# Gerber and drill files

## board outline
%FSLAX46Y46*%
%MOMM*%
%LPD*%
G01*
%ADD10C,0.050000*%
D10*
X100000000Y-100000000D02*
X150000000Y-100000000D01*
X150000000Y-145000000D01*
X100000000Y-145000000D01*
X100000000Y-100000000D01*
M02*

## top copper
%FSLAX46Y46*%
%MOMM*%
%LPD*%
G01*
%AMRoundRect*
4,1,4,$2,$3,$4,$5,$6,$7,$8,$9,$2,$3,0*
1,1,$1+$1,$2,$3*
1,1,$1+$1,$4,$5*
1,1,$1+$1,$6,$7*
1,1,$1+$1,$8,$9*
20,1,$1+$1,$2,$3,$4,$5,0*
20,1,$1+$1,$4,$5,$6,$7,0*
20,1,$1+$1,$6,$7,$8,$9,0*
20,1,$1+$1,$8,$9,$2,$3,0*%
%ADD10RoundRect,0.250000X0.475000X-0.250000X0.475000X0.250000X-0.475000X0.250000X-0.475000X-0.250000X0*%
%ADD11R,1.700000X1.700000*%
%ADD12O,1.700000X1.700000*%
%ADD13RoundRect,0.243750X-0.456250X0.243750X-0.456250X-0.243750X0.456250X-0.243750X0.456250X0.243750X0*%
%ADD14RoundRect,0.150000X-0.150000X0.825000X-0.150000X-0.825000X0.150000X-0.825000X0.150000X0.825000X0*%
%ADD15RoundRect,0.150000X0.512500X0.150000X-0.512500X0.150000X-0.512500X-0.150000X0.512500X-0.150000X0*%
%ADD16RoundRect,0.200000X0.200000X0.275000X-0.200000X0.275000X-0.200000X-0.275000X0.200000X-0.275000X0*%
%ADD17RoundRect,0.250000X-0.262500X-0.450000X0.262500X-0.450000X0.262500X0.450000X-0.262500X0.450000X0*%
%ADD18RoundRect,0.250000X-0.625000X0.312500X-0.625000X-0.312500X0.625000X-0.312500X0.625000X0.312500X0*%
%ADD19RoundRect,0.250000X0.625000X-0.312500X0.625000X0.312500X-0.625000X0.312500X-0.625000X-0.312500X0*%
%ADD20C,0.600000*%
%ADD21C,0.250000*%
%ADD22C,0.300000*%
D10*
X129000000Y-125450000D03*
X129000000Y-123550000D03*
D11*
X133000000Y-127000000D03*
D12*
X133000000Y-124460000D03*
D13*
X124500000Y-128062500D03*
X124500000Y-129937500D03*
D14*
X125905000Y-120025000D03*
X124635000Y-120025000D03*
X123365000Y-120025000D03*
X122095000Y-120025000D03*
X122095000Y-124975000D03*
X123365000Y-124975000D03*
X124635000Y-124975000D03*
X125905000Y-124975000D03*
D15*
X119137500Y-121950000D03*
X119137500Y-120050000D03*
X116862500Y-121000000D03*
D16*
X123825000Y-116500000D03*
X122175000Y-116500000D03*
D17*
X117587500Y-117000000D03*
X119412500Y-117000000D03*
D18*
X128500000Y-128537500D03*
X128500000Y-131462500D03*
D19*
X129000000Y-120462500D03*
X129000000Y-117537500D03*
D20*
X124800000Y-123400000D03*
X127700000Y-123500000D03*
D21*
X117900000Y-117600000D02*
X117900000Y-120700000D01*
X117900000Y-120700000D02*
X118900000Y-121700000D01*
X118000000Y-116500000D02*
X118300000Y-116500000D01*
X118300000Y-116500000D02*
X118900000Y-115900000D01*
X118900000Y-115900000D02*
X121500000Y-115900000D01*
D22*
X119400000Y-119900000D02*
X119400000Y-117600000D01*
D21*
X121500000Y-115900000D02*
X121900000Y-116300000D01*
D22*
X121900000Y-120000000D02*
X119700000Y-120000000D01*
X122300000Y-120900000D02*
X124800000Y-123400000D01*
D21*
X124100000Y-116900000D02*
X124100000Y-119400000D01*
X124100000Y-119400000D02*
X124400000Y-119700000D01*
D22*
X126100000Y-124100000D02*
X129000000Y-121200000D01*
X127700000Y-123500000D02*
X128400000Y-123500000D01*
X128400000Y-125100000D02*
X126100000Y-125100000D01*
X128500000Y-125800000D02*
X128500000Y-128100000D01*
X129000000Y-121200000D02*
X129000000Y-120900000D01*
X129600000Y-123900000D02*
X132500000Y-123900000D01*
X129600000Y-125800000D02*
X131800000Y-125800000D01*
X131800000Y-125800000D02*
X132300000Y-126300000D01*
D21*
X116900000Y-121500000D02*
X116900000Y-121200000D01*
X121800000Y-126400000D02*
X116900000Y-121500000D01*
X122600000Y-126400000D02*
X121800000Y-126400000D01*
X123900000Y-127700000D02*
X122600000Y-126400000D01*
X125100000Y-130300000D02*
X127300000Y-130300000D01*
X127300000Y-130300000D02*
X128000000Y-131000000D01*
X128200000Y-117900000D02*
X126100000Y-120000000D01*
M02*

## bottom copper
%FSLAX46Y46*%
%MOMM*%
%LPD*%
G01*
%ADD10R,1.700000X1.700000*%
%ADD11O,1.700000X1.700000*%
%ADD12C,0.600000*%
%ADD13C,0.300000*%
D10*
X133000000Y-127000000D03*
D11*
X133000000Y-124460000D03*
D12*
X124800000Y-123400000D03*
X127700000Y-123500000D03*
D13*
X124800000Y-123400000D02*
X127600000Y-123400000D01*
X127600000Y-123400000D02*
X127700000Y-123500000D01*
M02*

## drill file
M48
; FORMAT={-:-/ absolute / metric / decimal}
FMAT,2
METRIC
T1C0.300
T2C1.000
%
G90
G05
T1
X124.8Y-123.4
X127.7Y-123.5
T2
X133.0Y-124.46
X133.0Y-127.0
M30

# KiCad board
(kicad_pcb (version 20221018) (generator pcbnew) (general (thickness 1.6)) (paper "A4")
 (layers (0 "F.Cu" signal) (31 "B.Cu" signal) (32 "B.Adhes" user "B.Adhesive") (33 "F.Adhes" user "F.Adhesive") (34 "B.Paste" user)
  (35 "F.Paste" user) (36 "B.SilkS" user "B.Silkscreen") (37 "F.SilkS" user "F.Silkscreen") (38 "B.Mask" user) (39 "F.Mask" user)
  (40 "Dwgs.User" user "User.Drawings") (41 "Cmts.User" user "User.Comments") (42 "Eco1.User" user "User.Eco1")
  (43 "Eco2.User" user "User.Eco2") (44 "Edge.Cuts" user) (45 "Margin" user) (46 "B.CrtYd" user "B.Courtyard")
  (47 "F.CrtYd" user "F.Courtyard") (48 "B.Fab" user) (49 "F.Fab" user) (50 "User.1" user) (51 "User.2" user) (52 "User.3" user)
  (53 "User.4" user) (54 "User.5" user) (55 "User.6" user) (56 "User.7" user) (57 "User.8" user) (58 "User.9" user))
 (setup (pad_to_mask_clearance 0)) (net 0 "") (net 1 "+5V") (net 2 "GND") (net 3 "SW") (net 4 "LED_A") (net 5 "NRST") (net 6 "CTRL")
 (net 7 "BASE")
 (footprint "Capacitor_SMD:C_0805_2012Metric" (layer "F.Cu") (at 129 124.5 90)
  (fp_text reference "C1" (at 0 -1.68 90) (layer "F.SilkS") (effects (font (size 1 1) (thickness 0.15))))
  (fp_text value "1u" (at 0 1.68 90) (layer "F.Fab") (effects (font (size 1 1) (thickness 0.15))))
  (pad "1" smd roundrect (at -0.95 0 90) (size 1 1.45) (layers "F.Cu" "F.Paste" "F.Mask") (roundrect_rratio 0.25) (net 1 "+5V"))
  (pad "2" smd roundrect (at 0.95 0 90) (size 1 1.45) (layers "F.Cu" "F.Paste" "F.Mask") (roundrect_rratio 0.25) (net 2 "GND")))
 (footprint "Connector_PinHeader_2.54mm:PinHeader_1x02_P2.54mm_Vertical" (layer "F.Cu") (at 133 127 180)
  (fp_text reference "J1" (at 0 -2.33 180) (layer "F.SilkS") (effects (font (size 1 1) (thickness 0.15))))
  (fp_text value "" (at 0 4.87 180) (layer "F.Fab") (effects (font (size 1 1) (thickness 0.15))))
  (pad "1" thru_hole rect (at 0 0 180) (size 1.7 1.7) (drill 1) (layers "*.Cu" "*.Mask") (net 1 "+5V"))
  (pad "2" thru_hole oval (at 0 2.54 180) (size 1.7 1.7) (drill 1) (layers "*.Cu" "*.Mask") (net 2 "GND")))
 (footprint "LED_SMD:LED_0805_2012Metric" (layer "F.Cu") (at 124.5 129 -90)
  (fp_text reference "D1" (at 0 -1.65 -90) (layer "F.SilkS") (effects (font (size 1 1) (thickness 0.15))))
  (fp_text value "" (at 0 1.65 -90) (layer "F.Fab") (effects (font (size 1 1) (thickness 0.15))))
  (pad "1" smd roundrect (at -0.9375 0 270) (size 0.975 1.4) (layers "F.Cu" "F.Paste" "F.Mask") (roundrect_rratio 0.25) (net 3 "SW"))
  (pad "2" smd roundrect (at 0.9375 0 270) (size 0.975 1.4) (layers "F.Cu" "F.Paste" "F.Mask") (roundrect_rratio 0.25) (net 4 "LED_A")))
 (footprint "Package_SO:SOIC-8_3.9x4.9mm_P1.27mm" (layer "F.Cu") (at 124 122.5 -90)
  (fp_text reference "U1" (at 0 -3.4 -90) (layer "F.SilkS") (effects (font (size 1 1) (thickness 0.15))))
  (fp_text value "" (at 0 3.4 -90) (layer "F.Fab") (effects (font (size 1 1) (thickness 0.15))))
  (pad "1" smd roundrect (at -2.475 -1.905 270) (size 1.95 0.6) (layers "F.Cu" "F.Paste" "F.Mask") (roundrect_rratio 0.25) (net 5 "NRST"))
  (pad "2" smd roundrect (at -2.475 -0.635 270) (size 1.95 0.6) (layers "F.Cu" "F.Paste" "F.Mask") (roundrect_rratio 0.25) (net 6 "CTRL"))
  (pad "3" smd roundrect (at -2.475 0.635 270) (size 1.95 0.6) (layers "F.Cu" "F.Paste" "F.Mask") (roundrect_rratio 0.25))
  (pad "4" smd roundrect (at -2.475 1.905 270) (size 1.95 0.6) (layers "F.Cu" "F.Paste" "F.Mask") (roundrect_rratio 0.25) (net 2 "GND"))
  (pad "5" smd roundrect (at 2.475 1.905 270) (size 1.95 0.6) (layers "F.Cu" "F.Paste" "F.Mask") (roundrect_rratio 0.25))
  (pad "6" smd roundrect (at 2.475 0.635 270) (size 1.95 0.6) (layers "F.Cu" "F.Paste" "F.Mask") (roundrect_rratio 0.25))
  (pad "7" smd roundrect (at 2.475 -0.635 270) (size 1.95 0.6) (layers "F.Cu" "F.Paste" "F.Mask") (roundrect_rratio 0.25))
  (pad "8" smd roundrect (at 2.475 -1.905 270) (size 1.95 0.6) (layers "F.Cu" "F.Paste" "F.Mask") (roundrect_rratio 0.25) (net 1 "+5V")))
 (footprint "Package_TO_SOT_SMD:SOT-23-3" (layer "F.Cu") (at 118 121 180)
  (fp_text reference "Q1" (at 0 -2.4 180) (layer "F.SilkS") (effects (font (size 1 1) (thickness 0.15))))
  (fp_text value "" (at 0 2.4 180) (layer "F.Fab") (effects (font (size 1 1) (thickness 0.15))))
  (pad "1" smd roundrect (at -1.1375 -0.95 180) (size 1.325 0.6) (layers "F.Cu" "F.Paste" "F.Mask") (roundrect_rratio 0.25) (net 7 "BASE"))
  (pad "2" smd roundrect (at -1.1375 0.95 180) (size 1.325 0.6) (layers "F.Cu" "F.Paste" "F.Mask") (roundrect_rratio 0.25) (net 2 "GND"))
  (pad "3" smd roundrect (at 1.1375 0 180) (size 1.325 0.6) (layers "F.Cu" "F.Paste" "F.Mask") (roundrect_rratio 0.25) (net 3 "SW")))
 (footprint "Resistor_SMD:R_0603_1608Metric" (layer "F.Cu") (at 123 116.5 180)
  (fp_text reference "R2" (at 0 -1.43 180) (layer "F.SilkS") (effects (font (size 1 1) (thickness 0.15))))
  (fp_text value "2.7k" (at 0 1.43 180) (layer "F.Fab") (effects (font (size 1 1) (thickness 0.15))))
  (pad "1" smd roundrect (at -0.825 0 180) (size 0.8 0.95) (layers "F.Cu" "F.Paste" "F.Mask") (roundrect_rratio 0.25) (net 6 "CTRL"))
  (pad "2" smd roundrect (at 0.825 0 180) (size 0.8 0.95) (layers "F.Cu" "F.Paste" "F.Mask") (roundrect_rratio 0.25) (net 7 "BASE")))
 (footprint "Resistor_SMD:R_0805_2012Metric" (layer "F.Cu") (at 118.5 117)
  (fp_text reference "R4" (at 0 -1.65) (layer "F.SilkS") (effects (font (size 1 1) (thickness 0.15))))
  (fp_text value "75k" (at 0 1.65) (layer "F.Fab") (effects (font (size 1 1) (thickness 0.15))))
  (pad "1" smd roundrect (at -0.9125 0) (size 1.025 1.4) (layers "F.Cu" "F.Paste" "F.Mask") (roundrect_rratio 0.243902) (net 7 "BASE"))
  (pad "2" smd roundrect (at 0.9125 0) (size 1.025 1.4) (layers "F.Cu" "F.Paste" "F.Mask") (roundrect_rratio 0.243902) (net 2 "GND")))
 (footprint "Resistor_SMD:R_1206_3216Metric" (layer "F.Cu") (at 128.5 130 -90)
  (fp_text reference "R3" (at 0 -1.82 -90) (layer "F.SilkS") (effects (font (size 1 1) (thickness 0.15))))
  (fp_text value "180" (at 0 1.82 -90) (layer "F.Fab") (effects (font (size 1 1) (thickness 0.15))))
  (pad "1" smd roundrect (at -1.4625 0 270) (size 1.125 1.75) (layers "F.Cu" "F.Paste" "F.Mask") (roundrect_rratio 0.222222) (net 1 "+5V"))
  (pad "2" smd roundrect (at 1.4625 0 270) (size 1.125 1.75) (layers "F.Cu" "F.Paste" "F.Mask") (roundrect_rratio 0.222222) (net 4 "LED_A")))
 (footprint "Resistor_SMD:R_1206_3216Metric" (layer "F.Cu") (at 129 119 90)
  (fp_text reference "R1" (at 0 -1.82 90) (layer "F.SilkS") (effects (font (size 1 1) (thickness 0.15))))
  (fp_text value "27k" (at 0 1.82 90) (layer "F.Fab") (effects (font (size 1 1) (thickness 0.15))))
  (pad "1" smd roundrect (at -1.4625 0 90) (size 1.125 1.75) (layers "F.Cu" "F.Paste" "F.Mask") (roundrect_rratio 0.222222) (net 1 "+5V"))
  (pad "2" smd roundrect (at 1.4625 0 90) (size 1.125 1.75) (layers "F.Cu" "F.Paste" "F.Mask") (roundrect_rratio 0.222222) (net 5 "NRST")))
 (gr_rect (start 100 100) (end 150 145) (stroke (width 0.05) (type default)) (fill none) (layer "Edge.Cuts"))
 (segment (start 117.9 117.6) (end 117.9 120.7) (width 0.25) (layer "F.Cu") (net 7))
 (segment (start 117.9 120.7) (end 118.9 121.7) (width 0.25) (layer "F.Cu") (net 7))
 (segment (start 118 116.5) (end 118.3 116.5) (width 0.25) (layer "F.Cu") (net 7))
 (segment (start 118.3 116.5) (end 118.9 115.9) (width 0.25) (layer "F.Cu") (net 7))
 (segment (start 118.9 115.9) (end 121.5 115.9) (width 0.25) (layer "F.Cu") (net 7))
 (segment (start 119.4 119.9) (end 119.4 117.6) (width 0.3) (layer "F.Cu") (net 2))
 (segment (start 121.5 115.9) (end 121.9 116.3) (width 0.25) (layer "F.Cu") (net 7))
 (segment (start 121.9 120) (end 119.7 120) (width 0.3) (layer "F.Cu") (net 2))
 (segment (start 122.3 120.9) (end 124.8 123.4) (width 0.3) (layer "F.Cu") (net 2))
 (segment (start 124.1 116.9) (end 124.1 119.4) (width 0.25) (layer "F.Cu") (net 6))
 (segment (start 124.1 119.4) (end 124.4 119.7) (width 0.25) (layer "F.Cu") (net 6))
 (segment (start 126.1 124.1) (end 129 121.2) (width 0.3) (layer "F.Cu") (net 1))
 (segment (start 127.7 123.5) (end 128.4 123.5) (width 0.3) (layer "F.Cu") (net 2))
 (segment (start 128.4 125.1) (end 126.1 125.1) (width 0.3) (layer "F.Cu") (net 1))
 (segment (start 128.5 125.8) (end 128.5 128.1) (width 0.3) (layer "F.Cu") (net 1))
 (segment (start 129 121.2) (end 129 120.9) (width 0.3) (layer "F.Cu") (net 1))
 (segment (start 129.6 123.9) (end 132.5 123.9) (width 0.3) (layer "F.Cu") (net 2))
 (segment (start 129.6 125.8) (end 131.8 125.8) (width 0.3) (layer "F.Cu") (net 1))
 (segment (start 131.8 125.8) (end 132.3 126.3) (width 0.3) (layer "F.Cu") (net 1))
 (via (at 124.8 123.4) (size 0.6) (drill 0.3) (layers "F.Cu" "B.Cu") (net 2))
 (via (at 127.7 123.5) (size 0.6) (drill 0.3) (layers "F.Cu" "B.Cu") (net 2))
 (segment (start 116.9 121.5) (end 116.9 121.2) (width 0.25) (layer "F.Cu") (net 3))
 (segment (start 121.8 126.4) (end 116.9 121.5) (width 0.25) (layer "F.Cu") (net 3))
 (segment (start 122.6 126.4) (end 121.8 126.4) (width 0.25) (layer "F.Cu") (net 3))
 (segment (start 123.9 127.7) (end 122.6 126.4) (width 0.25) (layer "F.Cu") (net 3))
 (segment (start 124.8 123.4) (end 127.6 123.4) (width 0.3) (layer "B.Cu") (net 2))
 (segment (start 125.1 130.3) (end 127.3 130.3) (width 0.25) (layer "F.Cu") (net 4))
 (segment (start 127.3 130.3) (end 128 131) (width 0.25) (layer "F.Cu") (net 4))
 (segment (start 127.6 123.4) (end 127.7 123.5) (width 0.3) (layer "B.Cu") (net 2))
 (segment (start 128.2 117.9) (end 126.1 120) (width 0.25) (layer "F.Cu") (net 5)))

